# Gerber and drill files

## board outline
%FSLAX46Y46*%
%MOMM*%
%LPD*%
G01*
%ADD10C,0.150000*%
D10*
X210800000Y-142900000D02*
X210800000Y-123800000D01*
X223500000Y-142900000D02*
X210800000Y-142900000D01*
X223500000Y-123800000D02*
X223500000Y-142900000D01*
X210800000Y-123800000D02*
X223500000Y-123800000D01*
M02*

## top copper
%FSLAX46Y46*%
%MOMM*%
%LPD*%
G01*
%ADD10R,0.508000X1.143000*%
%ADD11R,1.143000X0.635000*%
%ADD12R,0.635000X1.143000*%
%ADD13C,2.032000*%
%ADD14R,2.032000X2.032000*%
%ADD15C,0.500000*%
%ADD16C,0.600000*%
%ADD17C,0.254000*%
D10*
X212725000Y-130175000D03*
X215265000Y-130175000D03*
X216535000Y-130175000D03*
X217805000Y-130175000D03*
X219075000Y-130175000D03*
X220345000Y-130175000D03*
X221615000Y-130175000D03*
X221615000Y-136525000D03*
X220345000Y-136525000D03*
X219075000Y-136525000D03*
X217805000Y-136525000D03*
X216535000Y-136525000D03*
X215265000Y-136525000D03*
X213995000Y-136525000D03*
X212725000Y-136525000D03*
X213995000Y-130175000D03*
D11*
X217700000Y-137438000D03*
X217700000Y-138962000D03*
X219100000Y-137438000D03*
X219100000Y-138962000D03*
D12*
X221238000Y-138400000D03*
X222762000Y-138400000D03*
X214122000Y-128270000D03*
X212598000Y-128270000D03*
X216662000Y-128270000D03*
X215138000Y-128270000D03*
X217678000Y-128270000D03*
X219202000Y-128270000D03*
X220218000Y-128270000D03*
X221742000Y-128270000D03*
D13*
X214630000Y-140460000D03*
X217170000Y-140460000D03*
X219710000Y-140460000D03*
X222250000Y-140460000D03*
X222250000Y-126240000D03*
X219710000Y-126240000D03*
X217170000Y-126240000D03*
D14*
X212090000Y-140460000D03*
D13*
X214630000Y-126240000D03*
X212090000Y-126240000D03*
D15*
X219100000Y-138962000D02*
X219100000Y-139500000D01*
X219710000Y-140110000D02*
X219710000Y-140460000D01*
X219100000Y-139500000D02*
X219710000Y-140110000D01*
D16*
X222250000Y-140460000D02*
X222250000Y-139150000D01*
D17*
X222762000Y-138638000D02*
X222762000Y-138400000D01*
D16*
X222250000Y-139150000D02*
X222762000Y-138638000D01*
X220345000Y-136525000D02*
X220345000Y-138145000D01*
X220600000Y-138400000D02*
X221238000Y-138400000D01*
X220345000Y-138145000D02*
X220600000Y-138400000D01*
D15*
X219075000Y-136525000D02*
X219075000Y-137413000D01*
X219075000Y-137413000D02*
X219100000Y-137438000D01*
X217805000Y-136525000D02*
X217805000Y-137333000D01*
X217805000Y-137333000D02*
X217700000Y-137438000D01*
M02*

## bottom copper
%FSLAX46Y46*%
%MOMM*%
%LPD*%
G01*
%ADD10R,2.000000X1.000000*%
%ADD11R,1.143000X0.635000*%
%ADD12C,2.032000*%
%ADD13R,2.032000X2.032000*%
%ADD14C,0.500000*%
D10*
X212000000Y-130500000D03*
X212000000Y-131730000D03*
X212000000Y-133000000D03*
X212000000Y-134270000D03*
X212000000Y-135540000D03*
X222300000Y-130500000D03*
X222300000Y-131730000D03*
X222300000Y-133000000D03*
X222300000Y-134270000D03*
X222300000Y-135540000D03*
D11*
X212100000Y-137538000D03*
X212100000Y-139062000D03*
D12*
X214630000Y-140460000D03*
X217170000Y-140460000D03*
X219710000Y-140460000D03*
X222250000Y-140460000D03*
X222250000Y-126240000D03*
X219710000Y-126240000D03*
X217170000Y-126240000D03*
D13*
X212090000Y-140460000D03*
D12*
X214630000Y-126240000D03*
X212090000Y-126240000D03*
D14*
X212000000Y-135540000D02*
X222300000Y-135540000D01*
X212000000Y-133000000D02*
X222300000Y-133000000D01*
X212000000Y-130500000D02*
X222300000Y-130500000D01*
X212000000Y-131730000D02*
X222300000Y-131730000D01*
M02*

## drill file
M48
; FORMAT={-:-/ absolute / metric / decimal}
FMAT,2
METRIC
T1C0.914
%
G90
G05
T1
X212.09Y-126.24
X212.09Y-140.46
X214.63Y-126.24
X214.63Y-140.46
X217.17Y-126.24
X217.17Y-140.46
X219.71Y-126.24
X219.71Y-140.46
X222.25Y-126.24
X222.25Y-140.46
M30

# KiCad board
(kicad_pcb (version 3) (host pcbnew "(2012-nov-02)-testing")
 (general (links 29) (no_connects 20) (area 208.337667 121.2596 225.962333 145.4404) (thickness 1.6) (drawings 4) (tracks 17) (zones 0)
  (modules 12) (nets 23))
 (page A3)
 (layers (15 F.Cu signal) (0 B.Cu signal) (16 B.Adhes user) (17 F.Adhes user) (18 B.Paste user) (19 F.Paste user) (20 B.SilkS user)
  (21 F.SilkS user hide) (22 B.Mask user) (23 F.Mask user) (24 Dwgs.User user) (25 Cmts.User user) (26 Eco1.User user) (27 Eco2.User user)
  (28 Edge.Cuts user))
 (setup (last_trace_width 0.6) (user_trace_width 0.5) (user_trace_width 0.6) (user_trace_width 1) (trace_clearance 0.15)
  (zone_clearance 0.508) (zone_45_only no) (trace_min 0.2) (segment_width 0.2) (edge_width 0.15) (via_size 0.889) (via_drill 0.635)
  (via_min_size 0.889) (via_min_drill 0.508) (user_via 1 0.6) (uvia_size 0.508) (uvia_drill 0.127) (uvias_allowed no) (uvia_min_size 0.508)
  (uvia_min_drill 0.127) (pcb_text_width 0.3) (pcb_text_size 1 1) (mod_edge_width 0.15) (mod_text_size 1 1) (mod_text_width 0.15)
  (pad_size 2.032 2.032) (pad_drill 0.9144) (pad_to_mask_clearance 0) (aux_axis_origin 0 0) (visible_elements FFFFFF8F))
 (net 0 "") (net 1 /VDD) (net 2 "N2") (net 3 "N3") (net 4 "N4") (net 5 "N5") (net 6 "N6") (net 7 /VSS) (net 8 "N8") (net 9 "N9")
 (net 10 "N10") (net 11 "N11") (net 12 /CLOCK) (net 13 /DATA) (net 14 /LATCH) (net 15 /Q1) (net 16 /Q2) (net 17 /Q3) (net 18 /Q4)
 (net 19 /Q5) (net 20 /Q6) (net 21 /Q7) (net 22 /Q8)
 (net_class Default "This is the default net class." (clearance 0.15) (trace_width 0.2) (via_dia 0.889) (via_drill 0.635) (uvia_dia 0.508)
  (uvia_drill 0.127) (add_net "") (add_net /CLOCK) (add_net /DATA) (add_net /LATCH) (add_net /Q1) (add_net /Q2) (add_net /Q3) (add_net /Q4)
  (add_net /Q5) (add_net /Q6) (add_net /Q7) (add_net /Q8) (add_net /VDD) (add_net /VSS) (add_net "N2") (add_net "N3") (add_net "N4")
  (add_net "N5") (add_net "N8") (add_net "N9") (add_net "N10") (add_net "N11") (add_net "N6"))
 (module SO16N (layer F.Cu) (at 217.17 133.35)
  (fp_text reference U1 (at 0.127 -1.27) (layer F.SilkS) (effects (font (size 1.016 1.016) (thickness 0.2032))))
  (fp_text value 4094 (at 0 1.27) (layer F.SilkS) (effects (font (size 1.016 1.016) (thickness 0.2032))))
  (pad 16 smd rect (at -4.445 -3.175) (size 0.508 1.143) (layers F.Cu F.Paste F.Mask) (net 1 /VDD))
  (pad 14 smd rect (at -1.905 -3.175) (size 0.508 1.143) (layers F.Cu F.Paste F.Mask) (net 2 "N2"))
  (pad 13 smd rect (at -0.635 -3.175) (size 0.508 1.143) (layers F.Cu F.Paste F.Mask) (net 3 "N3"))
  (pad 12 smd rect (at 0.635 -3.175) (size 0.508 1.143) (layers F.Cu F.Paste F.Mask) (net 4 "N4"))
  (pad 11 smd rect (at 1.905 -3.175) (size 0.508 1.143) (layers F.Cu F.Paste F.Mask) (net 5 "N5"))
  (pad 10 smd rect (at 3.175 -3.175) (size 0.508 1.143) (layers F.Cu F.Paste F.Mask) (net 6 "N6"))
  (pad 9 smd rect (at 4.445 -3.175) (size 0.508 1.143) (layers F.Cu F.Paste F.Mask))
  (pad 8 smd rect (at 4.445 3.175) (size 0.508 1.143) (layers F.Cu F.Paste F.Mask) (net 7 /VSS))
  (pad 7 smd rect (at 3.175 3.175) (size 0.508 1.143) (layers F.Cu F.Paste F.Mask) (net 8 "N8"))
  (pad 6 smd rect (at 1.905 3.175) (size 0.508 1.143) (layers F.Cu F.Paste F.Mask) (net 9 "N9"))
  (pad 5 smd rect (at 0.635 3.175) (size 0.508 1.143) (layers F.Cu F.Paste F.Mask) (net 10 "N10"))
  (pad 4 smd rect (at -0.635 3.175) (size 0.508 1.143) (layers F.Cu F.Paste F.Mask) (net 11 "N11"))
  (pad 3 smd rect (at -1.905 3.175) (size 0.508 1.143) (layers F.Cu F.Paste F.Mask) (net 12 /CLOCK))
  (pad 2 smd rect (at -3.175 3.175) (size 0.508 1.143) (layers F.Cu F.Paste F.Mask) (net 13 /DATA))
  (pad 1 smd rect (at -4.445 3.175) (size 0.508 1.143) (layers F.Cu F.Paste F.Mask) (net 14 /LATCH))
  (pad 15 smd rect (at -3.175 -3.175) (size 0.508 1.143) (layers F.Cu F.Paste F.Mask) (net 1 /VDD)))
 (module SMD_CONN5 (layer B.Cu) (at 212 133 180)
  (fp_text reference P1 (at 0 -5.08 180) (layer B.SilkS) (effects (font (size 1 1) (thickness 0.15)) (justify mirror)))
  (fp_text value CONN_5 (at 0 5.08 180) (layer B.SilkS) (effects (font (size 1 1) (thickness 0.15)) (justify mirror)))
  (pad 1 smd rect (at 0 2.5 180) (size 2 1) (layers B.Cu B.Paste B.Mask) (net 1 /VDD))
  (pad 2 smd rect (at 0 1.27 180) (size 2 1) (layers B.Cu B.Paste B.Mask) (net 7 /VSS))
  (pad 3 smd rect (at 0 0 180) (size 2 1) (layers B.Cu B.Paste B.Mask) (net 14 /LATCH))
  (pad 4 smd rect (at 0 -1.27 180) (size 2 1) (layers B.Cu B.Paste B.Mask) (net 13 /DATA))
  (pad 5 smd rect (at 0 -2.54 180) (size 2 1) (layers B.Cu B.Paste B.Mask) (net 12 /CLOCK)))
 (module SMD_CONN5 (layer B.Cu) (at 222.3 133 180)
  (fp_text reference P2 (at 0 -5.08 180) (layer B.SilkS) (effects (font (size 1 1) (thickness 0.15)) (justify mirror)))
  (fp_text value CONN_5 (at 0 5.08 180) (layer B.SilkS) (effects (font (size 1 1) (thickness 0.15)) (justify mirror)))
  (pad 1 smd rect (at 0 2.5 180) (size 2 1) (layers B.Cu B.Paste B.Mask) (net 1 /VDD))
  (pad 2 smd rect (at 0 1.27 180) (size 2 1) (layers B.Cu B.Paste B.Mask) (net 7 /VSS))
  (pad 3 smd rect (at 0 0 180) (size 2 1) (layers B.Cu B.Paste B.Mask) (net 14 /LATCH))
  (pad 4 smd rect (at 0 -1.27 180) (size 2 1) (layers B.Cu B.Paste B.Mask) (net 6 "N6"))
  (pad 5 smd rect (at 0 -2.54 180) (size 2 1) (layers B.Cu B.Paste B.Mask) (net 12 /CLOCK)))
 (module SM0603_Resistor (layer B.Cu) (at 212.1 138.3 270)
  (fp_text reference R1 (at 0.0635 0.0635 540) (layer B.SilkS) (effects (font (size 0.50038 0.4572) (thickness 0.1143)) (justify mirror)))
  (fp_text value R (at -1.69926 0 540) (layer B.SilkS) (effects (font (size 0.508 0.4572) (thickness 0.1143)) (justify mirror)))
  (pad 1 smd rect (at -0.762 0 270) (size 0.635 1.143) (layers B.Cu B.Paste B.Mask) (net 11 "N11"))
  (pad 2 smd rect (at 0.762 0 270) (size 0.635 1.143) (layers B.Cu B.Paste B.Mask) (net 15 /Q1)))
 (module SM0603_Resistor (layer F.Cu) (at 217.7 138.2 270)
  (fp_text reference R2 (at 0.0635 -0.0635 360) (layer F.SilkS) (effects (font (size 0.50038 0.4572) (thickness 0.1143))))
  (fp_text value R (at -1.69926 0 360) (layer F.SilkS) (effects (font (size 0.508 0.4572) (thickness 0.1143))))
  (pad 1 smd rect (at -0.762 0 270) (size 0.635 1.143) (layers F.Cu F.Paste F.Mask) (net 10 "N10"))
  (pad 2 smd rect (at 0.762 0 270) (size 0.635 1.143) (layers F.Cu F.Paste F.Mask) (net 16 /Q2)))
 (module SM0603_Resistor (layer F.Cu) (at 219.1 138.2 270)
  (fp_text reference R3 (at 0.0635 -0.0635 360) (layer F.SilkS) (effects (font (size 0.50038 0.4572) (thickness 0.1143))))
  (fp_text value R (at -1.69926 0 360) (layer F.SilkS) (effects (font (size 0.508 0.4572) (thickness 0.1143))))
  (pad 1 smd rect (at -0.762 0 270) (size 0.635 1.143) (layers F.Cu F.Paste F.Mask) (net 9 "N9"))
  (pad 2 smd rect (at 0.762 0 270) (size 0.635 1.143) (layers F.Cu F.Paste F.Mask) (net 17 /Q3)))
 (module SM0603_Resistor (layer F.Cu) (at 222 138.4)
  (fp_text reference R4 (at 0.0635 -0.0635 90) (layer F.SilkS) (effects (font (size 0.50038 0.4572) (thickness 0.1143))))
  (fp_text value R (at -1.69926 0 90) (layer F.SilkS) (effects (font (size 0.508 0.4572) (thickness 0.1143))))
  (pad 1 smd rect (at -0.762 0) (size 0.635 1.143) (layers F.Cu F.Paste F.Mask) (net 8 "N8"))
  (pad 2 smd rect (at 0.762 0) (size 0.635 1.143) (layers F.Cu F.Paste F.Mask) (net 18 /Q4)))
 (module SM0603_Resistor (layer F.Cu) (at 213.36 128.27 180)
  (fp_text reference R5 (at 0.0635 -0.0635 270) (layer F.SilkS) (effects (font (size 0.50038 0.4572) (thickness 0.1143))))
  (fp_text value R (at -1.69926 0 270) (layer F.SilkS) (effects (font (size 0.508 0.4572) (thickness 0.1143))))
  (pad 1 smd rect (at -0.762 0 180) (size 0.635 1.143) (layers F.Cu F.Paste F.Mask) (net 2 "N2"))
  (pad 2 smd rect (at 0.762 0 180) (size 0.635 1.143) (layers F.Cu F.Paste F.Mask) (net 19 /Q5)))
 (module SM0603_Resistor (layer F.Cu) (at 215.9 128.27 180)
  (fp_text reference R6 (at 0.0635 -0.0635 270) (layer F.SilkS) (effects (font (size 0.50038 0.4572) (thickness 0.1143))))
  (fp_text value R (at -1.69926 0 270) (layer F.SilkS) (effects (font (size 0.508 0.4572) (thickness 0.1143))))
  (pad 1 smd rect (at -0.762 0 180) (size 0.635 1.143) (layers F.Cu F.Paste F.Mask) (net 3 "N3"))
  (pad 2 smd rect (at 0.762 0 180) (size 0.635 1.143) (layers F.Cu F.Paste F.Mask) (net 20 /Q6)))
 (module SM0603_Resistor (layer F.Cu) (at 218.44 128.27)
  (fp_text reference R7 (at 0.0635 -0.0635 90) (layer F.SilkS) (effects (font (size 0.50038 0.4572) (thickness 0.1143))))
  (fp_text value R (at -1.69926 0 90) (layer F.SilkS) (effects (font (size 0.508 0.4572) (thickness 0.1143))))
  (pad 1 smd rect (at -0.762 0) (size 0.635 1.143) (layers F.Cu F.Paste F.Mask) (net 4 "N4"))
  (pad 2 smd rect (at 0.762 0) (size 0.635 1.143) (layers F.Cu F.Paste F.Mask) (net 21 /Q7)))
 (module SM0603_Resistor (layer F.Cu) (at 220.98 128.27)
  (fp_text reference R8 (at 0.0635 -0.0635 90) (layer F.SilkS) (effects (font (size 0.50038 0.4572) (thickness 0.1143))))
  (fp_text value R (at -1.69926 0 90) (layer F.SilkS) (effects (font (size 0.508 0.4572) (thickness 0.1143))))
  (pad 1 smd rect (at -0.762 0) (size 0.635 1.143) (layers F.Cu F.Paste F.Mask) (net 5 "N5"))
  (pad 2 smd rect (at 0.762 0) (size 0.635 1.143) (layers F.Cu F.Paste F.Mask) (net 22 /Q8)))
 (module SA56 (layer F.Cu) (at 217.17 133.35)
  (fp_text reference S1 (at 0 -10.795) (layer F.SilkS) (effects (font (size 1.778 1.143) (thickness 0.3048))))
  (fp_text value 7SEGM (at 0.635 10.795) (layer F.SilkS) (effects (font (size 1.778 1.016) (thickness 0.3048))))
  (pad 2 thru_hole circle (at -2.54 7.11) (size 2.032 2.032) (drill 0.9144) (layers *.Cu *.Mask F.SilkS) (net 16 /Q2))
  (pad 3 thru_hole circle (at 0 7.11) (size 2.032 2.032) (drill 0.9144) (layers *.Cu *.Mask F.SilkS) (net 1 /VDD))
  (pad 4 thru_hole circle (at 2.54 7.11) (size 2.032 2.032) (drill 0.9144) (layers *.Cu *.Mask F.SilkS) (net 17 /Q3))
  (pad 5 thru_hole circle (at 5.08 7.11) (size 2.032 2.032) (drill 0.9144) (layers *.Cu *.Mask F.SilkS) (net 18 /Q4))
  (pad 6 thru_hole circle (at 5.08 -7.11) (size 2.032 2.032) (drill 0.9144) (layers *.Cu *.Mask F.SilkS) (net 22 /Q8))
  (pad 7 thru_hole circle (at 2.54 -7.11) (size 2.032 2.032) (drill 0.9144) (layers *.Cu *.Mask F.SilkS) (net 21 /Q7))
  (pad 8 thru_hole circle (at 0 -7.11) (size 2.032 2.032) (drill 0.9144) (layers *.Cu *.Mask F.SilkS) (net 1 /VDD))
  (pad 1 thru_hole rect (at -5.08 7.11) (size 2.032 2.032) (drill 0.9144) (layers *.Cu *.Mask F.SilkS) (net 15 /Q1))
  (pad 9 thru_hole circle (at -2.54 -7.11) (size 2.032 2.032) (drill 0.9144) (layers *.Cu *.Mask F.SilkS) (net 20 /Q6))
  (pad 10 thru_hole circle (at -5.08 -7.11) (size 2.032 2.032) (drill 0.9144) (layers *.Cu *.Mask F.SilkS) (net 19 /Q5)))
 (gr_line (start 210.8 142.9) (end 210.8 123.8) (angle 90) (layer Edge.Cuts) (width 0.15))
 (gr_line (start 223.5 142.9) (end 210.8 142.9) (angle 90) (layer Edge.Cuts) (width 0.15))
 (gr_line (start 223.5 123.8) (end 223.5 142.9) (angle 90) (layer Edge.Cuts) (width 0.15))
 (gr_line (start 210.8 123.8) (end 223.5 123.8) (angle 90) (layer Edge.Cuts) (width 0.15))
 (segment (start 212 135.54) (end 222.3 135.54) (width 0.5) (layer B.Cu) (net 12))
 (segment (start 212 133) (end 222.3 133) (width 0.5) (layer B.Cu) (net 14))
 (segment (start 219.1 138.962) (end 219.1 139.5) (width 0.5) (layer F.Cu) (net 17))
 (segment (start 219.71 140.11) (end 219.71 140.46) (width 0.5) (layer F.Cu) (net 17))
 (segment (start 219.1 139.5) (end 219.71 140.11) (width 0.5) (layer F.Cu) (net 17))
 (segment (start 222.25 140.46) (end 222.25 139.15) (width 0.6) (layer F.Cu) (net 18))
 (segment (start 222.762 138.638) (end 222.762 138.4) (width 0.254) (layer F.Cu) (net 18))
 (segment (start 222.25 139.15) (end 222.762 138.638) (width 0.6) (layer F.Cu) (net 18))
 (segment (start 212 130.5) (end 222.3 130.5) (width 0.5) (layer B.Cu) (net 1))
 (segment (start 212 131.73) (end 222.3 131.73) (width 0.5) (layer B.Cu) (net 7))
 (segment (start 220.345 136.525) (end 220.345 138.145) (width 0.6) (layer F.Cu) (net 8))
 (segment (start 220.6 138.4) (end 221.238 138.4) (width 0.6) (layer F.Cu) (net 8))
 (segment (start 220.345 138.145) (end 220.6 138.4) (width 0.6) (layer F.Cu) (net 8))
 (segment (start 219.075 136.525) (end 219.075 137.413) (width 0.5) (layer F.Cu) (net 9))
 (segment (start 219.075 137.413) (end 219.1 137.438) (width 0.5) (layer F.Cu) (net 9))
 (segment (start 217.805 136.525) (end 217.805 137.333) (width 0.5) (layer F.Cu) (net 10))
 (segment (start 217.805 137.333) (end 217.7 137.438) (width 0.5) (layer F.Cu) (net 10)))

